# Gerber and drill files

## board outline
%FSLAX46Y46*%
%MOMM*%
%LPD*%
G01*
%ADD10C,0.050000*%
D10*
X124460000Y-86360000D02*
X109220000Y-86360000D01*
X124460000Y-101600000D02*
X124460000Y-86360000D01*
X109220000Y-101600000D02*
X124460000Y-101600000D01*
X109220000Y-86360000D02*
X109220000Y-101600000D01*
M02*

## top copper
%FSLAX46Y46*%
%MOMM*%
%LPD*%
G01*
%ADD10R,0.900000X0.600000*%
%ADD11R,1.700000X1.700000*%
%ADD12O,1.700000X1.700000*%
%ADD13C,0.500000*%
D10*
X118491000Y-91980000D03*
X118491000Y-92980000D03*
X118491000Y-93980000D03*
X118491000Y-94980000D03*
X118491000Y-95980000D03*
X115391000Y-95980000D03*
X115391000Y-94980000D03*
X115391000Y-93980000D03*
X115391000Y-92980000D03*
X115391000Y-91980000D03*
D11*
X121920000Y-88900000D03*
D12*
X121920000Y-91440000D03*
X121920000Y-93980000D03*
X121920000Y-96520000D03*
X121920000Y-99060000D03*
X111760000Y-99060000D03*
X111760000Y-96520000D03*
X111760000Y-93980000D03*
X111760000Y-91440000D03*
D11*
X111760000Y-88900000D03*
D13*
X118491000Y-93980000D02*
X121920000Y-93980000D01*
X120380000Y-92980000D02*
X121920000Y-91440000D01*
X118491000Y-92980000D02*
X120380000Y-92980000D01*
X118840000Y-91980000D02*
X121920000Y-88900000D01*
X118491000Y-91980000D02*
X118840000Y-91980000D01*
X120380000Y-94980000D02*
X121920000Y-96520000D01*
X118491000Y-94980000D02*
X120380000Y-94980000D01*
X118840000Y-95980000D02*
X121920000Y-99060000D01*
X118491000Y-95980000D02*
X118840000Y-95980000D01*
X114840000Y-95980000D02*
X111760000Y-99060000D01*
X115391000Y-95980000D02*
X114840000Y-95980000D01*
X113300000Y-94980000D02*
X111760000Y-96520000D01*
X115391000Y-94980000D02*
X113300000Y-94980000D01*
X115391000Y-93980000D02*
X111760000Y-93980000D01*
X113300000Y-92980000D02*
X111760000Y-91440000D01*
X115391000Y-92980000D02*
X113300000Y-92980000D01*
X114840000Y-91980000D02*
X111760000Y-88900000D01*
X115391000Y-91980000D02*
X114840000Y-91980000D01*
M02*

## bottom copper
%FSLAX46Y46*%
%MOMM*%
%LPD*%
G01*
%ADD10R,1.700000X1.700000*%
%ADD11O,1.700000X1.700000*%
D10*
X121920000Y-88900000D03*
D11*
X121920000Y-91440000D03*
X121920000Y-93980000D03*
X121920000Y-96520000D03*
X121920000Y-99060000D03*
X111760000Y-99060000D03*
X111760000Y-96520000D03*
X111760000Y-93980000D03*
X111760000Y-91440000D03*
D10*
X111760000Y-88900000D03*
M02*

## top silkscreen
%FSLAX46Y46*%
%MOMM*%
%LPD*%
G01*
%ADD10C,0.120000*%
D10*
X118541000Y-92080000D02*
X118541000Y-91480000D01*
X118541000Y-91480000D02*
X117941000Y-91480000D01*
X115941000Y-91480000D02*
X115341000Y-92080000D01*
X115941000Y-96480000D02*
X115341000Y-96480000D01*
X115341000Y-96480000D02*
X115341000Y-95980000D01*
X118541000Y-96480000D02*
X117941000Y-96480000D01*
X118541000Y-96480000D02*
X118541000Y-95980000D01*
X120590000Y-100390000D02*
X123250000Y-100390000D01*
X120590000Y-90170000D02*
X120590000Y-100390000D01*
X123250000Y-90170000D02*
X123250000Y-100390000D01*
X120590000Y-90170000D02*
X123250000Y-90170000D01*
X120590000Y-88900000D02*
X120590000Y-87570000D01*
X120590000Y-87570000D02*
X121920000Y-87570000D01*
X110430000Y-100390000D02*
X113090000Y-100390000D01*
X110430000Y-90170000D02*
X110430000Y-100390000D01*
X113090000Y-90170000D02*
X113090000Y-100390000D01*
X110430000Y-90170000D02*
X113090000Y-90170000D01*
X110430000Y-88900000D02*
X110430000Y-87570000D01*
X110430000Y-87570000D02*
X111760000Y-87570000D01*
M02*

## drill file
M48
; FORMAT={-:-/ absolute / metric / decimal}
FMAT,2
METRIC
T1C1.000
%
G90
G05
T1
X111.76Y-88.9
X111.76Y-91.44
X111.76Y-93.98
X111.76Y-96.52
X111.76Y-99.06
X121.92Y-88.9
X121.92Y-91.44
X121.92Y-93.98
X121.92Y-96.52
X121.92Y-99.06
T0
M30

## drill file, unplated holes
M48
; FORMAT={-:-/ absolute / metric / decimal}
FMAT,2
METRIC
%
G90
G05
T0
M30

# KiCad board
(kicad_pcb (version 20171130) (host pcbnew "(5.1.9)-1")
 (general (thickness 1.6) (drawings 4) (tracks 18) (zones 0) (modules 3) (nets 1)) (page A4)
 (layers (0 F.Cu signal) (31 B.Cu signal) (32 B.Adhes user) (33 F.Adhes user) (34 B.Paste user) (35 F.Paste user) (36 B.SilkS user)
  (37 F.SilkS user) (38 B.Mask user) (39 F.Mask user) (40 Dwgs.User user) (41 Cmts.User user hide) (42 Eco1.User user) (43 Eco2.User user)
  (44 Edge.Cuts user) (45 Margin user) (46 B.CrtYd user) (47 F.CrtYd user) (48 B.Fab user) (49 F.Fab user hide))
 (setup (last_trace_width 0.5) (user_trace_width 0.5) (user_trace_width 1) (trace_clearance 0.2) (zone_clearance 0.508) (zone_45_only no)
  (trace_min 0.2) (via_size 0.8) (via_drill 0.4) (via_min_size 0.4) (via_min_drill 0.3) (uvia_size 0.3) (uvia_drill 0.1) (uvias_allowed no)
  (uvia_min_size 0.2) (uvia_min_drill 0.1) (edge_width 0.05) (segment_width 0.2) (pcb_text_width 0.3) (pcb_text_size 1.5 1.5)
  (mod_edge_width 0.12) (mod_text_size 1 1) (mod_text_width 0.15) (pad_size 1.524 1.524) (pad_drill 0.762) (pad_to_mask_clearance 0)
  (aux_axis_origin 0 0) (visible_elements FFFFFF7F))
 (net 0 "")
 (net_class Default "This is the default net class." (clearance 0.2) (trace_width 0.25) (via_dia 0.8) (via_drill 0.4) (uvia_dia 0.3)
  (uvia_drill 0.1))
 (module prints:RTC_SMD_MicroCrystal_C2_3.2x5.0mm (layer F.Cu) (at 116.941 93.98)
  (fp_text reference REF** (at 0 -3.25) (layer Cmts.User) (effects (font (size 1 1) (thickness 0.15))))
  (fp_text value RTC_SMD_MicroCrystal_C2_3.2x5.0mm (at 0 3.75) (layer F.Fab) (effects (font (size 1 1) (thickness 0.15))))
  (fp_line (start 1.6 -1.9) (end 1.6 -2.5) (layer F.SilkS) (width 0.12))
  (fp_line (start 1.6 -2.5) (end 1 -2.5) (layer F.SilkS) (width 0.12))
  (fp_line (start -1 -2.5) (end -1.6 -1.9) (layer F.SilkS) (width 0.12))
  (fp_line (start -1 2.5) (end -1.6 2.5) (layer F.SilkS) (width 0.12))
  (fp_line (start -1.6 2.5) (end -1.6 2) (layer F.SilkS) (width 0.12))
  (fp_line (start 1.6 2.5) (end 1 2.5) (layer F.SilkS) (width 0.12))
  (fp_line (start 1.6 2.5) (end 1.6 2) (layer F.SilkS) (width 0.12))
  (pad 10 smd rect (at 1.55 -2) (size 0.9 0.6) (layers F.Cu F.Paste F.Mask))
  (pad 9 smd rect (at 1.55 -1) (size 0.9 0.6) (layers F.Cu F.Paste F.Mask))
  (pad 8 smd rect (at 1.55 0) (size 0.9 0.6) (layers F.Cu F.Paste F.Mask))
  (pad 7 smd rect (at 1.55 1) (size 0.9 0.6) (layers F.Cu F.Paste F.Mask))
  (pad 6 smd rect (at 1.55 2) (size 0.9 0.6) (layers F.Cu F.Paste F.Mask))
  (pad 5 smd rect (at -1.55 2) (size 0.9 0.6) (layers F.Cu F.Paste F.Mask))
  (pad 4 smd rect (at -1.55 1) (size 0.9 0.6) (layers F.Cu F.Paste F.Mask))
  (pad 3 smd rect (at -1.55 0) (size 0.9 0.6) (layers F.Cu F.Paste F.Mask))
  (pad 2 smd rect (at -1.55 -1) (size 0.9 0.6) (layers F.Cu F.Paste F.Mask))
  (pad 1 smd rect (at -1.55 -2) (size 0.9 0.6) (layers F.Cu F.Paste F.Mask)))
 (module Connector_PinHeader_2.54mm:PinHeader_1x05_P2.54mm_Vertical (layer F.Cu) (at 121.92 88.9)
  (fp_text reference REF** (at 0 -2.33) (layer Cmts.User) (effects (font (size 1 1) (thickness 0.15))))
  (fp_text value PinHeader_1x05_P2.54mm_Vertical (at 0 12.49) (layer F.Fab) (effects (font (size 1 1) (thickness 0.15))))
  (fp_line (start -1.33 11.49) (end 1.33 11.49) (layer F.SilkS) (width 0.12))
  (fp_line (start -1.33 1.27) (end -1.33 11.49) (layer F.SilkS) (width 0.12))
  (fp_line (start 1.33 1.27) (end 1.33 11.49) (layer F.SilkS) (width 0.12))
  (fp_line (start -1.33 1.27) (end 1.33 1.27) (layer F.SilkS) (width 0.12))
  (fp_line (start -1.33 0) (end -1.33 -1.33) (layer F.SilkS) (width 0.12))
  (fp_line (start -1.33 -1.33) (end 0 -1.33) (layer F.SilkS) (width 0.12))
  (pad 1 thru_hole rect (at 0 0) (size 1.7 1.7) (drill 1) (layers *.Cu *.Mask))
  (pad 2 thru_hole oval (at 0 2.54) (size 1.7 1.7) (drill 1) (layers *.Cu *.Mask))
  (pad 3 thru_hole oval (at 0 5.08) (size 1.7 1.7) (drill 1) (layers *.Cu *.Mask))
  (pad 4 thru_hole oval (at 0 7.62) (size 1.7 1.7) (drill 1) (layers *.Cu *.Mask))
  (pad 5 thru_hole oval (at 0 10.16) (size 1.7 1.7) (drill 1) (layers *.Cu *.Mask)))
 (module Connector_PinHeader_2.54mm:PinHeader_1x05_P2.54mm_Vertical (layer F.Cu) (at 111.76 88.9)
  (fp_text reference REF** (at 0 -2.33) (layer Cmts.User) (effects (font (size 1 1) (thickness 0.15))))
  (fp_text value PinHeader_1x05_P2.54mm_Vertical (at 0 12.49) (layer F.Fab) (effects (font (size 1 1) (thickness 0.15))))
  (fp_line (start -1.33 11.49) (end 1.33 11.49) (layer F.SilkS) (width 0.12))
  (fp_line (start -1.33 1.27) (end -1.33 11.49) (layer F.SilkS) (width 0.12))
  (fp_line (start 1.33 1.27) (end 1.33 11.49) (layer F.SilkS) (width 0.12))
  (fp_line (start -1.33 1.27) (end 1.33 1.27) (layer F.SilkS) (width 0.12))
  (fp_line (start -1.33 0) (end -1.33 -1.33) (layer F.SilkS) (width 0.12))
  (fp_line (start -1.33 -1.33) (end 0 -1.33) (layer F.SilkS) (width 0.12))
  (pad 5 thru_hole oval (at 0 10.16) (size 1.7 1.7) (drill 1) (layers *.Cu *.Mask))
  (pad 4 thru_hole oval (at 0 7.62) (size 1.7 1.7) (drill 1) (layers *.Cu *.Mask))
  (pad 3 thru_hole oval (at 0 5.08) (size 1.7 1.7) (drill 1) (layers *.Cu *.Mask))
  (pad 2 thru_hole oval (at 0 2.54) (size 1.7 1.7) (drill 1) (layers *.Cu *.Mask))
  (pad 1 thru_hole rect (at 0 0) (size 1.7 1.7) (drill 1) (layers *.Cu *.Mask)))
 (gr_line (start 124.46 86.36) (end 109.22 86.36) (layer Edge.Cuts) (width 0.05))
 (gr_line (start 124.46 101.6) (end 124.46 86.36) (layer Edge.Cuts) (width 0.05))
 (gr_line (start 109.22 101.6) (end 124.46 101.6) (layer Edge.Cuts) (width 0.05))
 (gr_line (start 109.22 86.36) (end 109.22 101.6) (layer Edge.Cuts) (width 0.05))
 (segment (start 118.491 93.98) (end 121.92 93.98) (width 0.5) (layer F.Cu) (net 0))
 (segment (start 120.38 92.98) (end 121.92 91.44) (width 0.5) (layer F.Cu) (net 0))
 (segment (start 118.491 92.98) (end 120.38 92.98) (width 0.5) (layer F.Cu) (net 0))
 (segment (start 118.84 91.98) (end 121.92 88.9) (width 0.5) (layer F.Cu) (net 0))
 (segment (start 118.491 91.98) (end 118.84 91.98) (width 0.5) (layer F.Cu) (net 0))
 (segment (start 120.38 94.98) (end 121.92 96.52) (width 0.5) (layer F.Cu) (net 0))
 (segment (start 118.491 94.98) (end 120.38 94.98) (width 0.5) (layer F.Cu) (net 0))
 (segment (start 118.84 95.98) (end 121.92 99.06) (width 0.5) (layer F.Cu) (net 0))
 (segment (start 118.491 95.98) (end 118.84 95.98) (width 0.5) (layer F.Cu) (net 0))
 (segment (start 114.84 95.98) (end 111.76 99.06) (width 0.5) (layer F.Cu) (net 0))
 (segment (start 115.391 95.98) (end 114.84 95.98) (width 0.5) (layer F.Cu) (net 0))
 (segment (start 113.3 94.98) (end 111.76 96.52) (width 0.5) (layer F.Cu) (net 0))
 (segment (start 115.391 94.98) (end 113.3 94.98) (width 0.5) (layer F.Cu) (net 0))
 (segment (start 115.391 93.98) (end 111.76 93.98) (width 0.5) (layer F.Cu) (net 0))
 (segment (start 113.3 92.98) (end 111.76 91.44) (width 0.5) (layer F.Cu) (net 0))
 (segment (start 115.391 92.98) (end 113.3 92.98) (width 0.5) (layer F.Cu) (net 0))
 (segment (start 114.84 91.98) (end 111.76 88.9) (width 0.5) (layer F.Cu) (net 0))
 (segment (start 115.391 91.98) (end 114.84 91.98) (width 0.5) (layer F.Cu) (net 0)))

